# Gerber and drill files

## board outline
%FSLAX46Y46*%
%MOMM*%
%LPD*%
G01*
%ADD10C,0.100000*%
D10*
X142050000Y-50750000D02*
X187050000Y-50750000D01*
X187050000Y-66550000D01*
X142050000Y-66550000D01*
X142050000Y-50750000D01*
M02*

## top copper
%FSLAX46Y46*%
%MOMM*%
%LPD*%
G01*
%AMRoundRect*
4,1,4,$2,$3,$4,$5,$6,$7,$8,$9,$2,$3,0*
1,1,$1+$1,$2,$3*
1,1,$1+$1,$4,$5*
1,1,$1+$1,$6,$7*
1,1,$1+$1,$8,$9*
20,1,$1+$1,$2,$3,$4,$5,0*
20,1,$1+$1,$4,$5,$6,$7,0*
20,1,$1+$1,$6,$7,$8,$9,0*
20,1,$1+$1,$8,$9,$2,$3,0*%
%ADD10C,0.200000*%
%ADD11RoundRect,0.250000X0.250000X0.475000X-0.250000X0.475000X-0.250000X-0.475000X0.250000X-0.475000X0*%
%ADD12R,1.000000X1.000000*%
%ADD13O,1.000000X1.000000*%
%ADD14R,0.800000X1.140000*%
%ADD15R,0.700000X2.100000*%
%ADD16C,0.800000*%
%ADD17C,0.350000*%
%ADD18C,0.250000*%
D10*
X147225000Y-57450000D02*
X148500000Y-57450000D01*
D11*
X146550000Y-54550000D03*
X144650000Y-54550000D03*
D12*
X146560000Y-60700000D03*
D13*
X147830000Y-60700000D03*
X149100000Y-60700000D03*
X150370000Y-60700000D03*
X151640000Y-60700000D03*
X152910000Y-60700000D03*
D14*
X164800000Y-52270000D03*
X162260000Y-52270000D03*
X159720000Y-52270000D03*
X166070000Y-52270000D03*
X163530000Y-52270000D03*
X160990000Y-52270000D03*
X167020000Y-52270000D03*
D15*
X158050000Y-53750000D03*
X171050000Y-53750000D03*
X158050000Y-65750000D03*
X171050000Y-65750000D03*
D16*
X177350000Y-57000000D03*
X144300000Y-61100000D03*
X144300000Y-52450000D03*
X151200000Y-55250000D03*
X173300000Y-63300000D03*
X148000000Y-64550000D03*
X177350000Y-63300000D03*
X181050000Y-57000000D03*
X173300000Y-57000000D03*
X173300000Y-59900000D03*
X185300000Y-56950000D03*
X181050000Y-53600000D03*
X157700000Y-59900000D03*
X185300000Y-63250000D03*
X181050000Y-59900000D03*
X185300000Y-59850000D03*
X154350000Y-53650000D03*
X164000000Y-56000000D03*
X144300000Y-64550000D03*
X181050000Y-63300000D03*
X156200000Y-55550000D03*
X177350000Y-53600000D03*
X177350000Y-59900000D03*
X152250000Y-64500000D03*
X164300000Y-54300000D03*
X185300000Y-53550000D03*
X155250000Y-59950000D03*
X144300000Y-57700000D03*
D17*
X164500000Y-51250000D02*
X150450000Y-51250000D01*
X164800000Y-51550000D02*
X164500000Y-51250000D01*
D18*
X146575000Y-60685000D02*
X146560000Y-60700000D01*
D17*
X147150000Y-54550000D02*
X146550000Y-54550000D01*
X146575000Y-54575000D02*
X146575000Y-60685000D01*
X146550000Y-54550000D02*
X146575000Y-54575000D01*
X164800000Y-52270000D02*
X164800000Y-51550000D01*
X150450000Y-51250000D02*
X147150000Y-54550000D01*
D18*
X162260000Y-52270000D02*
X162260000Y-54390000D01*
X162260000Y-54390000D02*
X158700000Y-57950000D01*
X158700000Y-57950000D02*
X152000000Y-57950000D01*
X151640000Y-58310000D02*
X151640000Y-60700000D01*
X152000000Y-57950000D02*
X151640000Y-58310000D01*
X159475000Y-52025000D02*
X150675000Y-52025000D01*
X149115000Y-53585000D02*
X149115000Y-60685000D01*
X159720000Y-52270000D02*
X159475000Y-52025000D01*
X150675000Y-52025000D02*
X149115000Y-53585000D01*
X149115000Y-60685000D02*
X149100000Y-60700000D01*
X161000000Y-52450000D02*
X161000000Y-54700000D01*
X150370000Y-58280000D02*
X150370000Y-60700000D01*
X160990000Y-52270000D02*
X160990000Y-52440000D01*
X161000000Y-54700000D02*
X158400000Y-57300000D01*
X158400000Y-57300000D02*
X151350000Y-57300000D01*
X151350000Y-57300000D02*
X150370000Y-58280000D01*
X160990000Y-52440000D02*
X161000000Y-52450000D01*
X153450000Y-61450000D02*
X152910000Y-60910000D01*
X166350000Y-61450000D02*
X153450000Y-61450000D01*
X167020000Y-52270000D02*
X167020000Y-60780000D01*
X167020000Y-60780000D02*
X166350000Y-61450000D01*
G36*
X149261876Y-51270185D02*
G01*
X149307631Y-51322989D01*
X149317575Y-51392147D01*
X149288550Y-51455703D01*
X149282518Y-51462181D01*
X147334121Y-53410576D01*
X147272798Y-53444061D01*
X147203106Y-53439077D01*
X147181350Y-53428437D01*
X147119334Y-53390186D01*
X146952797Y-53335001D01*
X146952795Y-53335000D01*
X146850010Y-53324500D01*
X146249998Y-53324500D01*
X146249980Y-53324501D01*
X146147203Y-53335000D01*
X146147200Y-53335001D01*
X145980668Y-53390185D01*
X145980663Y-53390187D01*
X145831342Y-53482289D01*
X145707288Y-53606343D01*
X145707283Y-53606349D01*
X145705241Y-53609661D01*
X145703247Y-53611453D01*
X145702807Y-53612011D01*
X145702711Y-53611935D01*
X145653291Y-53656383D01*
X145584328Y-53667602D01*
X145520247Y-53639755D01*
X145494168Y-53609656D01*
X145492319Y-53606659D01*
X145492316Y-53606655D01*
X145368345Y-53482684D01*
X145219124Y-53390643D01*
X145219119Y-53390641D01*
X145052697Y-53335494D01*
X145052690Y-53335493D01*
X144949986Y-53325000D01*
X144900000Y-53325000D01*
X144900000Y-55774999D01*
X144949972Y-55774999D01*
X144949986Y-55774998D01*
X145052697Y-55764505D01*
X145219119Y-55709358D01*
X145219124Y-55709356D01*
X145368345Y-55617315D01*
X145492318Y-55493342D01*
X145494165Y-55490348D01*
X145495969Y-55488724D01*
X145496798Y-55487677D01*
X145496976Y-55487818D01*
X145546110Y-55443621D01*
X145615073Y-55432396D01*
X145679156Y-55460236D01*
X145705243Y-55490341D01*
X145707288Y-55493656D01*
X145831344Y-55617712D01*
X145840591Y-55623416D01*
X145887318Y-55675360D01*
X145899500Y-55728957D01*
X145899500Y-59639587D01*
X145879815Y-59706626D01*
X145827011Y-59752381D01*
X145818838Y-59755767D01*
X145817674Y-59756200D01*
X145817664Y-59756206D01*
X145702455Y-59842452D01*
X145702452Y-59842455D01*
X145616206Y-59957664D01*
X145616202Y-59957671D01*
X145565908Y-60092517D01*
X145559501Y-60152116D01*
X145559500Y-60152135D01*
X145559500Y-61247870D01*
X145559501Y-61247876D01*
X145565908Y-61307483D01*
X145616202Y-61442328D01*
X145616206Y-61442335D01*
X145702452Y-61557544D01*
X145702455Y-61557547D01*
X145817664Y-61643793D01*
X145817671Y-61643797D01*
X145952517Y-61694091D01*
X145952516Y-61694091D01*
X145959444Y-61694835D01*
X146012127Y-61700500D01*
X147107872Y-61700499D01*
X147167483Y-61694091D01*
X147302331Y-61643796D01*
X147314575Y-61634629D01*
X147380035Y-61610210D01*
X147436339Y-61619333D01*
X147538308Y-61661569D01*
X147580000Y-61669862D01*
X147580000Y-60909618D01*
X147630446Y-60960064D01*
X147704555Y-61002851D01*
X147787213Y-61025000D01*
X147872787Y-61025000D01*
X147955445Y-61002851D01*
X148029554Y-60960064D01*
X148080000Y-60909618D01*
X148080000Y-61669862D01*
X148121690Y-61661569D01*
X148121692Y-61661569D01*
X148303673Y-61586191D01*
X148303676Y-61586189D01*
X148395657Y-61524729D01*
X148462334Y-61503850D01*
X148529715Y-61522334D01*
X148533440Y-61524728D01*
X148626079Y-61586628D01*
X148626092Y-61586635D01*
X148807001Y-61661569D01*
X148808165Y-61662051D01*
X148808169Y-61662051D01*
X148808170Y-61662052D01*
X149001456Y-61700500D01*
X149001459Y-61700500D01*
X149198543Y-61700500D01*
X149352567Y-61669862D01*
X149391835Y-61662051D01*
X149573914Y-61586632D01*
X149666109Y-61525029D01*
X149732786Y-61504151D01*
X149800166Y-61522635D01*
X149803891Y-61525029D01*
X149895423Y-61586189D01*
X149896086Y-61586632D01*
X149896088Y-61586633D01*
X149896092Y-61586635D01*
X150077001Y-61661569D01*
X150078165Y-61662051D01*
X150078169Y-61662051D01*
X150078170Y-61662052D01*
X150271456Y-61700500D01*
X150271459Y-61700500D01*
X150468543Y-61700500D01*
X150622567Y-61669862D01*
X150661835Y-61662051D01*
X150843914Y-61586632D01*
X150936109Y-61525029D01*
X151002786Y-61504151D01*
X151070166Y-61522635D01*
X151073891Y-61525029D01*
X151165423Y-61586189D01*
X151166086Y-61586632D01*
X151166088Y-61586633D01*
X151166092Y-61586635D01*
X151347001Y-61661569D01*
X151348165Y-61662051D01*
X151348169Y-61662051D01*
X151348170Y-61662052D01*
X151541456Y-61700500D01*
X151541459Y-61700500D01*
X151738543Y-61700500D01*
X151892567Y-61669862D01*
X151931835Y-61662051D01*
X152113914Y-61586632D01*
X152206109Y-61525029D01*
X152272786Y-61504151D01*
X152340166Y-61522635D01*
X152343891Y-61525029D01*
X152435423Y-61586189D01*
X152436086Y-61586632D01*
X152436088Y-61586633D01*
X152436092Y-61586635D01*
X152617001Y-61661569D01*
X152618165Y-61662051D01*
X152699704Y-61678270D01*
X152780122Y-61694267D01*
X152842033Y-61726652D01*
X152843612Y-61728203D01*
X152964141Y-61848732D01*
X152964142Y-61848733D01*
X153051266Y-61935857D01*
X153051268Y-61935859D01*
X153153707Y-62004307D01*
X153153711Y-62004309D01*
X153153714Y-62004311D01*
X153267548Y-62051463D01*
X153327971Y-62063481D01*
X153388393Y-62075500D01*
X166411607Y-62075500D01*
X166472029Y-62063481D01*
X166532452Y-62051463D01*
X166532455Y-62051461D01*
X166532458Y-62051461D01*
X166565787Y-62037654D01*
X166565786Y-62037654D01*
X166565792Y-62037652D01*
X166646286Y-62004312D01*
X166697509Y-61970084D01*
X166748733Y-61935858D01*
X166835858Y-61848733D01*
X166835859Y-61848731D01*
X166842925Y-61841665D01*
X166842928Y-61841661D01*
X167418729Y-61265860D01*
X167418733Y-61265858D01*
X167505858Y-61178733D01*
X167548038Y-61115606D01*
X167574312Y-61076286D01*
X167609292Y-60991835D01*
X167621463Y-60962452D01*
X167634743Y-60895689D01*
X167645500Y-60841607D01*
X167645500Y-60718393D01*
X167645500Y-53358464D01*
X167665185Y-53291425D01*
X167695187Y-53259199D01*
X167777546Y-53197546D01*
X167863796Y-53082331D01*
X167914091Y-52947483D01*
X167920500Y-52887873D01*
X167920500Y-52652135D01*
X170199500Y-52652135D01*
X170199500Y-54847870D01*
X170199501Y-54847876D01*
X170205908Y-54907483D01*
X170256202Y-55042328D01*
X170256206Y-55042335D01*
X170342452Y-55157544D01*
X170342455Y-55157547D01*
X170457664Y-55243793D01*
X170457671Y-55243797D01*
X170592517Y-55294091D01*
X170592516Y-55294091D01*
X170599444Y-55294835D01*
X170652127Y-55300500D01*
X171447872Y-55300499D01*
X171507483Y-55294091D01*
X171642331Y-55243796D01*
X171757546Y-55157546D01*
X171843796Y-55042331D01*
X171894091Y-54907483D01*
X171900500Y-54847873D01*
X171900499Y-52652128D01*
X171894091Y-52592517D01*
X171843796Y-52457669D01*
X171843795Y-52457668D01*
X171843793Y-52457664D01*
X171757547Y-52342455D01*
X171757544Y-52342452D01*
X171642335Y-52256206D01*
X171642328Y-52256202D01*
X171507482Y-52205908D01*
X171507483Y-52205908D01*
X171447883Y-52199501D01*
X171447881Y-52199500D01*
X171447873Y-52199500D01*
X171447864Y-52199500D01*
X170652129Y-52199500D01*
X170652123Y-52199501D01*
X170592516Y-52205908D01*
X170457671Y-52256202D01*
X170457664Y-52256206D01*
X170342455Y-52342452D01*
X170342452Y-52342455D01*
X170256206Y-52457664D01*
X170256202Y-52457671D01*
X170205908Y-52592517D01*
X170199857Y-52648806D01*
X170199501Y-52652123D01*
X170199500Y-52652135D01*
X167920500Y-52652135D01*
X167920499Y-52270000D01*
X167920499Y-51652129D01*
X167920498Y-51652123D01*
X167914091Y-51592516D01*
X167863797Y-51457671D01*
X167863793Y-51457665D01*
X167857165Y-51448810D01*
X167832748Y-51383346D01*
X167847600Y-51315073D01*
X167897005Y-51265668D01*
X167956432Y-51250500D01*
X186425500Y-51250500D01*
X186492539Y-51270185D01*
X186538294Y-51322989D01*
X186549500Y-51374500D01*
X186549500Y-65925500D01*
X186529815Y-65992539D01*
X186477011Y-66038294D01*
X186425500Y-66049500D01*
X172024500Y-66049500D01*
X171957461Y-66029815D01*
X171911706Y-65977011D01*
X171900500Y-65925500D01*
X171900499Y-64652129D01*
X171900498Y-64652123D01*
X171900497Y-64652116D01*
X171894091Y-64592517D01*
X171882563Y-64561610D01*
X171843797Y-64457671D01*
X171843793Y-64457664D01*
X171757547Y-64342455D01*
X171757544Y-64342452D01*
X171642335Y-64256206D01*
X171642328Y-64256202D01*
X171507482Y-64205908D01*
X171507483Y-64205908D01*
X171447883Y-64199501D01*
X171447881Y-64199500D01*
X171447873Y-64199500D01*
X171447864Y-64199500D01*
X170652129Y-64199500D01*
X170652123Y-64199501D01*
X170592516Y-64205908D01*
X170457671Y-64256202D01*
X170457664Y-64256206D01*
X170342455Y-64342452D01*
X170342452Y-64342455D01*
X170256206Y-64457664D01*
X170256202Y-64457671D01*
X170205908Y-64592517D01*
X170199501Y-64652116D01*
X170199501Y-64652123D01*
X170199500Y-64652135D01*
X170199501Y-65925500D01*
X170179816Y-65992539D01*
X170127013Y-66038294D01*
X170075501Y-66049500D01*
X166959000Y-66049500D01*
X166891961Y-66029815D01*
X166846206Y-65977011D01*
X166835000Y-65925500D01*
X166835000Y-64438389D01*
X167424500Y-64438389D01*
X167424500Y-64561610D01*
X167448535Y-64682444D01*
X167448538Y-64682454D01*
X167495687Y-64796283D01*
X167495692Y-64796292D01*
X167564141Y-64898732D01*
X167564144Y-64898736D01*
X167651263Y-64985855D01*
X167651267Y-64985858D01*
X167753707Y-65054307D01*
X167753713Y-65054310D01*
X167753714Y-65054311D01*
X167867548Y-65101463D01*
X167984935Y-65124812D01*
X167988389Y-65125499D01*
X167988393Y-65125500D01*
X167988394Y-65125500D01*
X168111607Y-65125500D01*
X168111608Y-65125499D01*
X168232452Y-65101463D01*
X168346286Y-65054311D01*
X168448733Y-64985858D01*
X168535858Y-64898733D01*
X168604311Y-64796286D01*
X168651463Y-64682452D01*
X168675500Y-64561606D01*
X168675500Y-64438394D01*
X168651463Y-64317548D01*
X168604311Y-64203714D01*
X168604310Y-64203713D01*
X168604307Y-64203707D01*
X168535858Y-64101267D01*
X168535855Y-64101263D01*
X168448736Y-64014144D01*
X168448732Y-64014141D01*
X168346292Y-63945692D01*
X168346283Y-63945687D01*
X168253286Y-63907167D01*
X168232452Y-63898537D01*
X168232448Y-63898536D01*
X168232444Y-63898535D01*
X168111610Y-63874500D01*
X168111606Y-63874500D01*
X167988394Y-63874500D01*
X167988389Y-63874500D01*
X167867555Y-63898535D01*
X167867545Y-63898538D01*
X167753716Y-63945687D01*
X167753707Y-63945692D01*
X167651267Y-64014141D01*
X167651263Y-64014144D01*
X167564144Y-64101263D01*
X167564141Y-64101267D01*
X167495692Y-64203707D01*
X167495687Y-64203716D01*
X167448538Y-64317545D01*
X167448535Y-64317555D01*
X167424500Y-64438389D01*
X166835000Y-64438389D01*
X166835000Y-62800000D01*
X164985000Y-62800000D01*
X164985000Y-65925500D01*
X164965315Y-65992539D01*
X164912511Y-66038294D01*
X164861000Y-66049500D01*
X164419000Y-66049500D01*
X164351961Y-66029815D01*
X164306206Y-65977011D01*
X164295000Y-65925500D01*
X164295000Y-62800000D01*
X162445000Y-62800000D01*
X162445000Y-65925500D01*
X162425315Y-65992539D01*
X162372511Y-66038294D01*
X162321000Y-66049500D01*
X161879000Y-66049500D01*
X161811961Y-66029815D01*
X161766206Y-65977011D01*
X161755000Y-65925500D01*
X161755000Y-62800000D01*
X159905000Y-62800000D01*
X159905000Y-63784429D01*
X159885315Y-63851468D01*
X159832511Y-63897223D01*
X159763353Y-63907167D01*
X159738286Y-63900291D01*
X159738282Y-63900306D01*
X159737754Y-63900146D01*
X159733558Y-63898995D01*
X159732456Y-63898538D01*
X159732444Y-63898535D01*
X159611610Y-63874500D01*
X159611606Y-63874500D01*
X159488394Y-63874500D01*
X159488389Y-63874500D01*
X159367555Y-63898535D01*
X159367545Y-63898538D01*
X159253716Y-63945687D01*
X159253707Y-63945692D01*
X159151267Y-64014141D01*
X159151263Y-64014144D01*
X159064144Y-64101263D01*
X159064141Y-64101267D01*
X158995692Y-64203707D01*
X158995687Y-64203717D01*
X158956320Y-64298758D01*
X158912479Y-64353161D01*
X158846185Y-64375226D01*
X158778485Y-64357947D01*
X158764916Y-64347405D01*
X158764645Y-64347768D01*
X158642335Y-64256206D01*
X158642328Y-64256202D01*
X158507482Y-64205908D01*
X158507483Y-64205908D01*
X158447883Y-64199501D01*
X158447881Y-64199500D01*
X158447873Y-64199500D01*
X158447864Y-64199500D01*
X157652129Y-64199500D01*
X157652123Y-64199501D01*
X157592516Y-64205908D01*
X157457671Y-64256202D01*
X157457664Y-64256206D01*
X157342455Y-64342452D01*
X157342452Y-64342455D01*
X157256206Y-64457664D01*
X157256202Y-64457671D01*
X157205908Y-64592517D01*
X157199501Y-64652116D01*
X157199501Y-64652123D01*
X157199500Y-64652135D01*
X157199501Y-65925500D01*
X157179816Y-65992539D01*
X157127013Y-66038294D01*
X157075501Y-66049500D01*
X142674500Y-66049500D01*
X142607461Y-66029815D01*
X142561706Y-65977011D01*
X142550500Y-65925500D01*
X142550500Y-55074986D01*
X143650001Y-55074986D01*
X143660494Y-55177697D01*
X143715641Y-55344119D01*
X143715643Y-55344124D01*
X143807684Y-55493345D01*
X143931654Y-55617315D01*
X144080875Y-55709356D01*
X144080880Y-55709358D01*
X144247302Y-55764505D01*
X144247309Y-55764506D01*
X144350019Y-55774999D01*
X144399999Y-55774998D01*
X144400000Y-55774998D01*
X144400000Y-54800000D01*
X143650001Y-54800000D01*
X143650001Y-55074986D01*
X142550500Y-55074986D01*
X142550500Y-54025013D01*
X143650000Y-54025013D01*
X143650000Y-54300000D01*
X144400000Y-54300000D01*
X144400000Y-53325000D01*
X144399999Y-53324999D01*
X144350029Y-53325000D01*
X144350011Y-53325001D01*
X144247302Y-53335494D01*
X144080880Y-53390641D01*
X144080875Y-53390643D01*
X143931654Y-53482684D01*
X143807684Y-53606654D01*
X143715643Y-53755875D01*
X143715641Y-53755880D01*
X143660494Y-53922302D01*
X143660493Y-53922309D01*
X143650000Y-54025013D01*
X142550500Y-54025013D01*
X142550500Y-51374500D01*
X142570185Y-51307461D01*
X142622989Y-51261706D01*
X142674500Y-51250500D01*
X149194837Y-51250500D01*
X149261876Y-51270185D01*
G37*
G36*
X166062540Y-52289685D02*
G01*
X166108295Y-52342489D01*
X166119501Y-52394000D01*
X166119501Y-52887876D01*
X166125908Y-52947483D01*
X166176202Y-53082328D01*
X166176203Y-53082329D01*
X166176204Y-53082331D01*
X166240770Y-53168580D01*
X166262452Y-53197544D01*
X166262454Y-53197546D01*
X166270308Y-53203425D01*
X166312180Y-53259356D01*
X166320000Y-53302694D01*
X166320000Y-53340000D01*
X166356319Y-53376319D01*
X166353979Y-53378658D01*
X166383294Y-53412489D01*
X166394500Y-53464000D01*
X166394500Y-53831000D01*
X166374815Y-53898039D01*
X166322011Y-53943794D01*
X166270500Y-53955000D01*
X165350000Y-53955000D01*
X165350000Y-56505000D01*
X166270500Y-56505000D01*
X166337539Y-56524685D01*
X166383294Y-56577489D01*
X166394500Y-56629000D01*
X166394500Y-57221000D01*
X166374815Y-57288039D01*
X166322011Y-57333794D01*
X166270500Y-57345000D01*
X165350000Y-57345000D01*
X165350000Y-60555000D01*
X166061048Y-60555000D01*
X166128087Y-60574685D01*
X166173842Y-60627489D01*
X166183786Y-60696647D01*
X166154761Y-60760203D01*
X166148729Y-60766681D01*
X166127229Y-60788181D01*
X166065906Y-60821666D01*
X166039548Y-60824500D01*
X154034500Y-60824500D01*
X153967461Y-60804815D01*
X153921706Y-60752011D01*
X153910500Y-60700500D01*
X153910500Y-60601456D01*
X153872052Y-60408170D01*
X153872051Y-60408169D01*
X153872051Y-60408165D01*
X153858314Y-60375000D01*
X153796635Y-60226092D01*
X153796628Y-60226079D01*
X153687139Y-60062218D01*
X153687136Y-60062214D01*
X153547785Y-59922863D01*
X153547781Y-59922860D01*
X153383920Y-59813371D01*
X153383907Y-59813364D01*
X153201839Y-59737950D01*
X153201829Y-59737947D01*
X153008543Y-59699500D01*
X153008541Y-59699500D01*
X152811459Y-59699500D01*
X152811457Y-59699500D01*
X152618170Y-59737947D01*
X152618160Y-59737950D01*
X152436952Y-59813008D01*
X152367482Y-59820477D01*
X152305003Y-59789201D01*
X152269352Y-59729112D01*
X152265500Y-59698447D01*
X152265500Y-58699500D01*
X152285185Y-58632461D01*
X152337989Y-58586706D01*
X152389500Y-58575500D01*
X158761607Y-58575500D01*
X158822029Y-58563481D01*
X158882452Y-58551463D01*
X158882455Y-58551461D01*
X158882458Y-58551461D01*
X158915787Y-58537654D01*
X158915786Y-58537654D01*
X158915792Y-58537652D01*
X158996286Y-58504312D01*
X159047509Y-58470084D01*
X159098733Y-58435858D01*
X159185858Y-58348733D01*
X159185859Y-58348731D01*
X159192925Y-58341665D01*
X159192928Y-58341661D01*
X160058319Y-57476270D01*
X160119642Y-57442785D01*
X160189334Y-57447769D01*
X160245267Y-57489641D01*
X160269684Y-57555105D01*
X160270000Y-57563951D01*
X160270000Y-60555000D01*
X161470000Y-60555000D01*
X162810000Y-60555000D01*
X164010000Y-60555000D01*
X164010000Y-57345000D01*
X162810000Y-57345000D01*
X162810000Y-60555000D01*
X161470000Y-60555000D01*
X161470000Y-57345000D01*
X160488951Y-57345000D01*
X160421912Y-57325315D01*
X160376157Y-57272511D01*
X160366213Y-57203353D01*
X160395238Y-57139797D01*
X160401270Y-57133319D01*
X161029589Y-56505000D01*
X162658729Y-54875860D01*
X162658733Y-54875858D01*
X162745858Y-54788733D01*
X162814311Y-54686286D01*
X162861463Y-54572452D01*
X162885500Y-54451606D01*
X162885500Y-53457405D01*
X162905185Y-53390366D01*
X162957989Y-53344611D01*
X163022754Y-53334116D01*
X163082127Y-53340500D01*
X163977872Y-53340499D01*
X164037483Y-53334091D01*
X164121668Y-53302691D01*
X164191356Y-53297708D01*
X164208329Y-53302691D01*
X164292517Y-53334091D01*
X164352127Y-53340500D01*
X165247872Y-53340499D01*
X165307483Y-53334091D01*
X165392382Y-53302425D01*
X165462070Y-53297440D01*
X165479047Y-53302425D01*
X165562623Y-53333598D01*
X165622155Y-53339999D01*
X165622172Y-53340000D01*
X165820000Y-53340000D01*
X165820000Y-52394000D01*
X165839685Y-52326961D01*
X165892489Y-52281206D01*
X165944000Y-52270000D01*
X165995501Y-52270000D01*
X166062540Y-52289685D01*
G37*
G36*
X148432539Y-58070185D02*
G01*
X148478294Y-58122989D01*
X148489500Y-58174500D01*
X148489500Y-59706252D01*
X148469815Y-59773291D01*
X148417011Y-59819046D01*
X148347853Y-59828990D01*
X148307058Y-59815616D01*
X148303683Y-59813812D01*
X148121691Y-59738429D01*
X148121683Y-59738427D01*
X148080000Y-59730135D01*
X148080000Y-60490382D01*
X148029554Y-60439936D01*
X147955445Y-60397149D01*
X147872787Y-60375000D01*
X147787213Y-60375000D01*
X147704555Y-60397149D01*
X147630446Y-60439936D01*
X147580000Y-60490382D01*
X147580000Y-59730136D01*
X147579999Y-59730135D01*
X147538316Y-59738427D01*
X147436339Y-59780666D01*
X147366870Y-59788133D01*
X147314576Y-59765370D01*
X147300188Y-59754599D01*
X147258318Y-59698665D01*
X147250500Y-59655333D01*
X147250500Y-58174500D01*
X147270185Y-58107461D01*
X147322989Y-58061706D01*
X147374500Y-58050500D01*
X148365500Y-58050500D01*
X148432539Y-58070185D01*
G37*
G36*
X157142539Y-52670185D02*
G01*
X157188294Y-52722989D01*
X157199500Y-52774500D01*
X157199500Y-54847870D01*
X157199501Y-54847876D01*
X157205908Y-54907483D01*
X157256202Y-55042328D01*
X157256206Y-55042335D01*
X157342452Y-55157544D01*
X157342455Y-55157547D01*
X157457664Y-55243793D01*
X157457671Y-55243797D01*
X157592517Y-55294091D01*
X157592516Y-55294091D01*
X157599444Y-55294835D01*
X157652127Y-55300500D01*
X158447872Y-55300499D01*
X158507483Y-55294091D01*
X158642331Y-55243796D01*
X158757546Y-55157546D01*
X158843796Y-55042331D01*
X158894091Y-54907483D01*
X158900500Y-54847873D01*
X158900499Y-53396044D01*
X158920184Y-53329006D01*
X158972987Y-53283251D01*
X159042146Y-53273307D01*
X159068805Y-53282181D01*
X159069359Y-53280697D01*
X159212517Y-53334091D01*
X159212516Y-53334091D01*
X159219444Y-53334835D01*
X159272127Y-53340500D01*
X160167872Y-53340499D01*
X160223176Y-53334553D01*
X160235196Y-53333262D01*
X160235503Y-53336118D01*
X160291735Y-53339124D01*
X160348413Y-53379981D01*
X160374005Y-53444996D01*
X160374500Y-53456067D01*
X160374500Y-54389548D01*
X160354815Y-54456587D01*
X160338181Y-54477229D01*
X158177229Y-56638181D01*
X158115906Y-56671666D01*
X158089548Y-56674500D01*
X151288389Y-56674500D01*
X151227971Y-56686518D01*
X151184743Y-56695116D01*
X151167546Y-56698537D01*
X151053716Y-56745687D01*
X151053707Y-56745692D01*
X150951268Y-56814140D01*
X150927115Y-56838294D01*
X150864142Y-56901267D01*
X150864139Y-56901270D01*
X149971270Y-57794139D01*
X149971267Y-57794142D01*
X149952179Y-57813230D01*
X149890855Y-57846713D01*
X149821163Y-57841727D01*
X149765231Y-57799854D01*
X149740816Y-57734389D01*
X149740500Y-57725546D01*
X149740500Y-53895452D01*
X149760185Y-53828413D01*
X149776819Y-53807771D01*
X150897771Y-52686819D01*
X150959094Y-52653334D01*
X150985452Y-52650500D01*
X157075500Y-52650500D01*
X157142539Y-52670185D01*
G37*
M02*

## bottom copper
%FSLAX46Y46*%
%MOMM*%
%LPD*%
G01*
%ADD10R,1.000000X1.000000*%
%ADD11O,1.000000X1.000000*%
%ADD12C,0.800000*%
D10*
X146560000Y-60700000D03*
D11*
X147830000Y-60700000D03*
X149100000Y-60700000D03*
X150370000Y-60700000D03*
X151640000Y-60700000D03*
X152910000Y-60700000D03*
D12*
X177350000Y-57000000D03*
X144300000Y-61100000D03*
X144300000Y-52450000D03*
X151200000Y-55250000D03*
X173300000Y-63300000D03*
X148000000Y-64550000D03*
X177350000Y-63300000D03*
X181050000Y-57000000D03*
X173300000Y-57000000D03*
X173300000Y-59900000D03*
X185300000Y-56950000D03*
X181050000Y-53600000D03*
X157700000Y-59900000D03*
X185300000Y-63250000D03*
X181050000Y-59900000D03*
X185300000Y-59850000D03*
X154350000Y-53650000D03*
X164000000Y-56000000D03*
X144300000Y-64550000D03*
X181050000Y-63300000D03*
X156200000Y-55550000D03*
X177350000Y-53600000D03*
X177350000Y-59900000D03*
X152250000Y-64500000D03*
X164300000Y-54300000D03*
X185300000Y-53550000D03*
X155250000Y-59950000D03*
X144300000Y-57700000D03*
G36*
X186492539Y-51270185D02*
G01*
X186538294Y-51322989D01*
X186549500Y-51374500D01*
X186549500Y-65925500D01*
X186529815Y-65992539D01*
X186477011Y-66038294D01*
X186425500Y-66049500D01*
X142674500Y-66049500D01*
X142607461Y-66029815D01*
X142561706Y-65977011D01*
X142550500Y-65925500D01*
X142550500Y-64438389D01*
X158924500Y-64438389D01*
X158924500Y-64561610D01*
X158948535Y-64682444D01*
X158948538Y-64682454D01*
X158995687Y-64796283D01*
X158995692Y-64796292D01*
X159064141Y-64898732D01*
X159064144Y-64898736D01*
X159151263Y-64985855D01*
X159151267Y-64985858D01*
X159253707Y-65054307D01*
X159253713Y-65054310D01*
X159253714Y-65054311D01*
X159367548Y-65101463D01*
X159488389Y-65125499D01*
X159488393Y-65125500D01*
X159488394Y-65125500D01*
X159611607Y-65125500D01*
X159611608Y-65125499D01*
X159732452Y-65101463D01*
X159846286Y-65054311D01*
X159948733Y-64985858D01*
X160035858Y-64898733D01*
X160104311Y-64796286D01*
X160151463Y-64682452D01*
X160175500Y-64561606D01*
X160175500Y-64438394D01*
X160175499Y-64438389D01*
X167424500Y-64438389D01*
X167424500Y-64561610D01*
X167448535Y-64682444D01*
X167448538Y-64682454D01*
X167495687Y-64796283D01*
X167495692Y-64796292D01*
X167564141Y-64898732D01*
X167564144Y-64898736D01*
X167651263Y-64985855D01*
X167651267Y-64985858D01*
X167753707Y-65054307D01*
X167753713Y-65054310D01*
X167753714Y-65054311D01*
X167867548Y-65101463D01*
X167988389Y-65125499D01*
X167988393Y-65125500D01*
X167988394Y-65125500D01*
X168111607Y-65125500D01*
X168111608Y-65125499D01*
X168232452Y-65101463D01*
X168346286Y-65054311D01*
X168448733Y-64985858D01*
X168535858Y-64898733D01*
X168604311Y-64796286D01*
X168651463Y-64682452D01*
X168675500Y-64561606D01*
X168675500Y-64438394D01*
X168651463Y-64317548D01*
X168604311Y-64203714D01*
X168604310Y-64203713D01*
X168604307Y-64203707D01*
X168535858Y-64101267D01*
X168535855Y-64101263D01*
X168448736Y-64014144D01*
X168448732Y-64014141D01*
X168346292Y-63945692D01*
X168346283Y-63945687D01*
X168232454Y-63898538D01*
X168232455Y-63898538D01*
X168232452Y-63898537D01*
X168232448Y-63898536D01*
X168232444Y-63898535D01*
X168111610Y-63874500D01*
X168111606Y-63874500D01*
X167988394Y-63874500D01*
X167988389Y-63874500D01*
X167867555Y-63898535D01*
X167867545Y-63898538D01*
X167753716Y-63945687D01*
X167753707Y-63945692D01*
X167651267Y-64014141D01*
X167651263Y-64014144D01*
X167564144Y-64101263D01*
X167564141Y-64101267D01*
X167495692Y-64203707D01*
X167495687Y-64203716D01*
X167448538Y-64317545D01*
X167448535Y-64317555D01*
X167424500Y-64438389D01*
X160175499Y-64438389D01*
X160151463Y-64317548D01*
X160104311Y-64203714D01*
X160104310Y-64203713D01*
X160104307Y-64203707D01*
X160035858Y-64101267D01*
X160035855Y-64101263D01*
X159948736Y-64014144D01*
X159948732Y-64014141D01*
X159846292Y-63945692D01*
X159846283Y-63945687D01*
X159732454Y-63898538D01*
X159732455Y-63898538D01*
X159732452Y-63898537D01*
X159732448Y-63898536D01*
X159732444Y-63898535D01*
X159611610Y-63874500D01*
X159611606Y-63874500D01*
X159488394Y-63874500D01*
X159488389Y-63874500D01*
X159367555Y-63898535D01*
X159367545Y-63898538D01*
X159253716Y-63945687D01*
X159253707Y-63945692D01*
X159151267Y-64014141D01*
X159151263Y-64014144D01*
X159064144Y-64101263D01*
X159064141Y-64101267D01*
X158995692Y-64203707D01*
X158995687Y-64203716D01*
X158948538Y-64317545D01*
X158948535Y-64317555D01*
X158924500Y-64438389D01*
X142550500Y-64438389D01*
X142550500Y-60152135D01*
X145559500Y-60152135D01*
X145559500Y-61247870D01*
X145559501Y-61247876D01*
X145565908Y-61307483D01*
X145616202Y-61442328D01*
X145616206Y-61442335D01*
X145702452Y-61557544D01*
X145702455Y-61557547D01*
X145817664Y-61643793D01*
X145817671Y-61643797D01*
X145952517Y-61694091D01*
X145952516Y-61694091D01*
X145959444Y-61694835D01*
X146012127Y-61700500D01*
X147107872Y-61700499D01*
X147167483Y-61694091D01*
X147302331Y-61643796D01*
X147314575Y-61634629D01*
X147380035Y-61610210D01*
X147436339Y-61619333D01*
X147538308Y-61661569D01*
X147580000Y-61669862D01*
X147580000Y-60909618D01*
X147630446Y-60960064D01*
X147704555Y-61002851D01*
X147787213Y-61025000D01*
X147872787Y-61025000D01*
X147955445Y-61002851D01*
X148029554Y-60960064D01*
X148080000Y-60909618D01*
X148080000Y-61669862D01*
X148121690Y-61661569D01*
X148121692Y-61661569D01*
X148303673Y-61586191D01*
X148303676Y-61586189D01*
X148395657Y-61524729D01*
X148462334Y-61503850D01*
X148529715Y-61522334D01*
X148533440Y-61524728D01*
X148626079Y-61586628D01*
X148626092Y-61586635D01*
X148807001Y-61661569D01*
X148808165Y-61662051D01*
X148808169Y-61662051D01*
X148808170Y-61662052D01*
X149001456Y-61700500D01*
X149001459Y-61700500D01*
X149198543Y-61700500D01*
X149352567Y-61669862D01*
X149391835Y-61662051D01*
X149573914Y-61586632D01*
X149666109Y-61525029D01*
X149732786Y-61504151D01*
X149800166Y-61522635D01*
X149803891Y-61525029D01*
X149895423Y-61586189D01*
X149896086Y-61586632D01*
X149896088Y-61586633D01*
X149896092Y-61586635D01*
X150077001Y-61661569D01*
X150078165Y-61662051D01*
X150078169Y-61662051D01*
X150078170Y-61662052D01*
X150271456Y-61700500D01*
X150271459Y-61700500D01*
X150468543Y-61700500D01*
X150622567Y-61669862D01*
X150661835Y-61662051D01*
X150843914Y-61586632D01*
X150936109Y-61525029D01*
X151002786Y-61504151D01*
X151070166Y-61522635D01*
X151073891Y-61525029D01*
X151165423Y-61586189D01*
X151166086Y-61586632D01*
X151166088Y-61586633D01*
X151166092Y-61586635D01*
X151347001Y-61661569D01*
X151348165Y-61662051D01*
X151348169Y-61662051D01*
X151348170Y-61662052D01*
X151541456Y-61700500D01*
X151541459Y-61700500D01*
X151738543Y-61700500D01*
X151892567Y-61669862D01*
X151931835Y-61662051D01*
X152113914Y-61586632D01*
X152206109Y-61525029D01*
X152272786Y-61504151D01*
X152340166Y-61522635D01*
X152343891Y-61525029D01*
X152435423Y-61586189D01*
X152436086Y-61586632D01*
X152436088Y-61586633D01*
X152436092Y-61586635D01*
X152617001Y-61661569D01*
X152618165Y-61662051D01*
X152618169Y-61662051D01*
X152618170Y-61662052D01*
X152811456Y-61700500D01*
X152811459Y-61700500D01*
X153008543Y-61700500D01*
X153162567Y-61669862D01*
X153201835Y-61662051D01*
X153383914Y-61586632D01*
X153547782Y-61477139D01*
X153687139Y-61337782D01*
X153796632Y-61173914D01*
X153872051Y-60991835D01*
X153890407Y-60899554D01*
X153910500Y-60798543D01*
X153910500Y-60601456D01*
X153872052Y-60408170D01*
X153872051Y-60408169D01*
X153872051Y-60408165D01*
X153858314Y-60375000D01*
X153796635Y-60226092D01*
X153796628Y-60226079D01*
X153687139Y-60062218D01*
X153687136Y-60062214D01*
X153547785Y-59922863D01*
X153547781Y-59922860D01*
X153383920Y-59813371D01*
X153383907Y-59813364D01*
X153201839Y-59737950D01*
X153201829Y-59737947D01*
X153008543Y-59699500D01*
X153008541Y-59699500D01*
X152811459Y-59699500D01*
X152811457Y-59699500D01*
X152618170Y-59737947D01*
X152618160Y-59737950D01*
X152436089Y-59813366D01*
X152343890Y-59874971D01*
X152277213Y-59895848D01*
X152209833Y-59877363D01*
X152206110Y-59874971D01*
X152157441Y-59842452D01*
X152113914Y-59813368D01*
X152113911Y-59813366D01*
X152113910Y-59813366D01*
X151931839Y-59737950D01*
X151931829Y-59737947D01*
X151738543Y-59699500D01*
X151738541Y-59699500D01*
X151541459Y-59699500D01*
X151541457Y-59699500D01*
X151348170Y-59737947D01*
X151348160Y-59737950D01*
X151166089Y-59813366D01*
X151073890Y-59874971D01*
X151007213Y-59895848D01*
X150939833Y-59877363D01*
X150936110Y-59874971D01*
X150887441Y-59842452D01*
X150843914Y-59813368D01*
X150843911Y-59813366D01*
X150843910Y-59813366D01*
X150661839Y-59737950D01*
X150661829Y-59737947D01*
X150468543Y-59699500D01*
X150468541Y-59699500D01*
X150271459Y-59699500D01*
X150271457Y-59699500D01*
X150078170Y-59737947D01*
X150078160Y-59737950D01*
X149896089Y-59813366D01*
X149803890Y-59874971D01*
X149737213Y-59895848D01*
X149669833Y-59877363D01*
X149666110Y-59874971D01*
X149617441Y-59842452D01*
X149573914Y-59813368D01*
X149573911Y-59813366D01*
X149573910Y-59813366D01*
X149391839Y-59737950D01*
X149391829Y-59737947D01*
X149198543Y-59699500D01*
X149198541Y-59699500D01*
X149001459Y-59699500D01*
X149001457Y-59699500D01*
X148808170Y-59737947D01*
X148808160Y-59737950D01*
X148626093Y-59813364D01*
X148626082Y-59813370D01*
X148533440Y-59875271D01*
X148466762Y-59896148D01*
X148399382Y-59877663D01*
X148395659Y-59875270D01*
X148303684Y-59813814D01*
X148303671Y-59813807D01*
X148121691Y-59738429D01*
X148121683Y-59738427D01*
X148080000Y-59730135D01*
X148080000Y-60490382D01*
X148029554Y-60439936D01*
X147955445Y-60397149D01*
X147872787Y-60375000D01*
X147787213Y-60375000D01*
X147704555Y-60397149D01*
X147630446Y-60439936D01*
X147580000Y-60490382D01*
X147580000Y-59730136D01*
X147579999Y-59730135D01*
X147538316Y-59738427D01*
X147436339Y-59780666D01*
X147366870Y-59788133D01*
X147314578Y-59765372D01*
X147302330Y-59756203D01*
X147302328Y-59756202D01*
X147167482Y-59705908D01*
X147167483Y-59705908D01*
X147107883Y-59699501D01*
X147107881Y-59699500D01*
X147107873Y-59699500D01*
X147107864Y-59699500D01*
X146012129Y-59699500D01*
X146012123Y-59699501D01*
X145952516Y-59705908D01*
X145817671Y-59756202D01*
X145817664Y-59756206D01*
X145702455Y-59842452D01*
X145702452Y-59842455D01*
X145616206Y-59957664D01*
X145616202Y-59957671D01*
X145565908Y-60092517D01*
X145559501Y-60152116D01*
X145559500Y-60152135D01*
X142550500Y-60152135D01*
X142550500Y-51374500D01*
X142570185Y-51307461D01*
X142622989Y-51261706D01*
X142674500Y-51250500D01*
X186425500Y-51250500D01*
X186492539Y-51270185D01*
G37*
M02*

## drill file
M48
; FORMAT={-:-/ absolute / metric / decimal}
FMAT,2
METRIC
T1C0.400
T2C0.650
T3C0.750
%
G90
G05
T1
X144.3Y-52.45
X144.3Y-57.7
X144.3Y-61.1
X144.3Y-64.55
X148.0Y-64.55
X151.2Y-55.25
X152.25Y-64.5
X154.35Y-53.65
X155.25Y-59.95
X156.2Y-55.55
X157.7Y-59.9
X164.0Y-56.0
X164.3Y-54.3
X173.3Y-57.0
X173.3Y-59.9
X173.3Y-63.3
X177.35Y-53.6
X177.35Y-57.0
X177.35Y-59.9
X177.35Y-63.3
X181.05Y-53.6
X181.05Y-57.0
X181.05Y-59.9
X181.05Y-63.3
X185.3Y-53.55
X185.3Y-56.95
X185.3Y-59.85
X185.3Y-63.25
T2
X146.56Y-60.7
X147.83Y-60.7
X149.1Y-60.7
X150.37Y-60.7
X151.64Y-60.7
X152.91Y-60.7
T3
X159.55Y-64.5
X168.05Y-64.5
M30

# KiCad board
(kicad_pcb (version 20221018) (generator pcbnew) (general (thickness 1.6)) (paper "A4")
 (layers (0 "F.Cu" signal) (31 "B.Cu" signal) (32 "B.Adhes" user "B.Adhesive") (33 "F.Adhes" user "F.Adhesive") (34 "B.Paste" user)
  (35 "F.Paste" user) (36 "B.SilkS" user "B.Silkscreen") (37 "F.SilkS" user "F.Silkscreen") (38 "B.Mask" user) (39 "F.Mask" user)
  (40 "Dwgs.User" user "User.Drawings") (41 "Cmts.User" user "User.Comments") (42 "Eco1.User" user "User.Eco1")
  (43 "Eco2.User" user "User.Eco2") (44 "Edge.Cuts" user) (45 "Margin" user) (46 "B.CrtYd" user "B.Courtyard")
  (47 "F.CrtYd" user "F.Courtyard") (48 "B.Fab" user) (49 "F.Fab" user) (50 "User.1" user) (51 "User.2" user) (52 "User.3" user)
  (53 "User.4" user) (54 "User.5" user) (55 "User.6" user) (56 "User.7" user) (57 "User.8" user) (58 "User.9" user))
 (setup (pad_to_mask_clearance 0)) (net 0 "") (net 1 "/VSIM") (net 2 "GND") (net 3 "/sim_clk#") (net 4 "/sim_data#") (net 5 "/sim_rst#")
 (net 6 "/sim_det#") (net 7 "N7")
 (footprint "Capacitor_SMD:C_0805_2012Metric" (layer "F.Cu") (at 145.6 54.55 180)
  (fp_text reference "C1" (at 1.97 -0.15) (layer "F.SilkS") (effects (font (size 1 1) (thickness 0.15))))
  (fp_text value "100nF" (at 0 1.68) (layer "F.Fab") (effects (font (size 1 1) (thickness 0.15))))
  (pad "1" smd roundrect (at -0.95 0 180) (size 1 1.45) (layers "F.Cu" "F.Paste" "F.Mask") (roundrect_rratio 0.25) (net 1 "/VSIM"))
  (pad "2" smd roundrect (at 0.95 0 180) (size 1 1.45) (layers "F.Cu" "F.Paste" "F.Mask") (roundrect_rratio 0.25) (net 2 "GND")))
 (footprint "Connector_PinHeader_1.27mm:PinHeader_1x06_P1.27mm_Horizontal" (layer "F.Cu") (at 146.56 60.7 90)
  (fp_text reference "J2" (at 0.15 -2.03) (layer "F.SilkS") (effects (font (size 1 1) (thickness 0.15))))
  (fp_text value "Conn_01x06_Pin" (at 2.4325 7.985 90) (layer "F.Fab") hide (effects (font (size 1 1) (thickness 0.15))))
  (pad "1" thru_hole rect (at 0 0 90) (size 1 1) (drill 0.65) (layers "*.Cu" "*.Mask") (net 1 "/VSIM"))
  (pad "2" thru_hole oval (at 0 1.27 90) (size 1 1) (drill 0.65) (layers "*.Cu" "*.Mask") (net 2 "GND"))
  (pad "3" thru_hole oval (at 0 2.54 90) (size 1 1) (drill 0.65) (layers "*.Cu" "*.Mask") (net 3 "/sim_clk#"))
  (pad "4" thru_hole oval (at 0 3.81 90) (size 1 1) (drill 0.65) (layers "*.Cu" "*.Mask") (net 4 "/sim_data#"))
  (pad "5" thru_hole oval (at 0 5.08 90) (size 1 1) (drill 0.65) (layers "*.Cu" "*.Mask") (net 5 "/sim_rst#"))
  (pad "6" thru_hole oval (at 0 6.35 90) (size 1 1) (drill 0.65) (layers "*.Cu" "*.Mask") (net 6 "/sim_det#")))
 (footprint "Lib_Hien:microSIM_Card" (layer "F.Cu") (at 164.55 59.64)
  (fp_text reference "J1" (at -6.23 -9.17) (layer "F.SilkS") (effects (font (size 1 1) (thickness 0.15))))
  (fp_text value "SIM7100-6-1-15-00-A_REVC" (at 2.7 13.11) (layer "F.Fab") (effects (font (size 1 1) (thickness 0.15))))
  (pad "" np_thru_hole circle (at -5 4.86) (size 0.75 0.75) (drill 0.75) (layers "*.Cu" "*.Mask"))
  (pad "" np_thru_hole circle (at 3.5 4.86) (size 0.75 0.75) (drill 0.75) (layers "*.Cu" "*.Mask"))
  (pad "C1" smd rect (at 0.25 -7.37) (size 0.8 1.14) (layers "F.Cu" "F.Paste" "F.Mask") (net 1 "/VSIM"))
  (pad "C2" smd rect (at -2.29 -7.37) (size 0.8 1.14) (layers "F.Cu" "F.Paste" "F.Mask") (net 5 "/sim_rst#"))
  (pad "C3" smd rect (at -4.83 -7.37) (size 0.8 1.14) (layers "F.Cu" "F.Paste" "F.Mask") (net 3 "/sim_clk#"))
  (pad "C5" smd rect (at 1.52 -7.37) (size 0.8 1.14) (layers "F.Cu" "F.Paste" "F.Mask") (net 2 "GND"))
  (pad "C6" smd rect (at -1.02 -7.37) (size 0.8 1.14) (layers "F.Cu" "F.Paste" "F.Mask") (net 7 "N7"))
  (pad "C7" smd rect (at -3.56 -7.37) (size 0.8 1.14) (layers "F.Cu" "F.Paste" "F.Mask") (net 4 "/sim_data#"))
  (pad "CD" smd rect (at 2.47 -7.37) (size 0.8 1.14) (layers "F.Cu" "F.Paste" "F.Mask") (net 6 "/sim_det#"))
  (pad "G1" smd rect (at -6.5 -5.89) (size 0.7 2.1) (layers "F.Cu" "F.Paste" "F.Mask"))
  (pad "G2" smd rect (at 6.5 -5.89) (size 0.7 2.1) (layers "F.Cu" "F.Paste" "F.Mask"))
  (pad "G3" smd rect (at -6.5 6.11) (size 0.7 2.1) (layers "F.Cu" "F.Paste" "F.Mask"))
  (pad "G4" smd rect (at 6.5 6.11) (size 0.7 2.1) (layers "F.Cu" "F.Paste" "F.Mask"))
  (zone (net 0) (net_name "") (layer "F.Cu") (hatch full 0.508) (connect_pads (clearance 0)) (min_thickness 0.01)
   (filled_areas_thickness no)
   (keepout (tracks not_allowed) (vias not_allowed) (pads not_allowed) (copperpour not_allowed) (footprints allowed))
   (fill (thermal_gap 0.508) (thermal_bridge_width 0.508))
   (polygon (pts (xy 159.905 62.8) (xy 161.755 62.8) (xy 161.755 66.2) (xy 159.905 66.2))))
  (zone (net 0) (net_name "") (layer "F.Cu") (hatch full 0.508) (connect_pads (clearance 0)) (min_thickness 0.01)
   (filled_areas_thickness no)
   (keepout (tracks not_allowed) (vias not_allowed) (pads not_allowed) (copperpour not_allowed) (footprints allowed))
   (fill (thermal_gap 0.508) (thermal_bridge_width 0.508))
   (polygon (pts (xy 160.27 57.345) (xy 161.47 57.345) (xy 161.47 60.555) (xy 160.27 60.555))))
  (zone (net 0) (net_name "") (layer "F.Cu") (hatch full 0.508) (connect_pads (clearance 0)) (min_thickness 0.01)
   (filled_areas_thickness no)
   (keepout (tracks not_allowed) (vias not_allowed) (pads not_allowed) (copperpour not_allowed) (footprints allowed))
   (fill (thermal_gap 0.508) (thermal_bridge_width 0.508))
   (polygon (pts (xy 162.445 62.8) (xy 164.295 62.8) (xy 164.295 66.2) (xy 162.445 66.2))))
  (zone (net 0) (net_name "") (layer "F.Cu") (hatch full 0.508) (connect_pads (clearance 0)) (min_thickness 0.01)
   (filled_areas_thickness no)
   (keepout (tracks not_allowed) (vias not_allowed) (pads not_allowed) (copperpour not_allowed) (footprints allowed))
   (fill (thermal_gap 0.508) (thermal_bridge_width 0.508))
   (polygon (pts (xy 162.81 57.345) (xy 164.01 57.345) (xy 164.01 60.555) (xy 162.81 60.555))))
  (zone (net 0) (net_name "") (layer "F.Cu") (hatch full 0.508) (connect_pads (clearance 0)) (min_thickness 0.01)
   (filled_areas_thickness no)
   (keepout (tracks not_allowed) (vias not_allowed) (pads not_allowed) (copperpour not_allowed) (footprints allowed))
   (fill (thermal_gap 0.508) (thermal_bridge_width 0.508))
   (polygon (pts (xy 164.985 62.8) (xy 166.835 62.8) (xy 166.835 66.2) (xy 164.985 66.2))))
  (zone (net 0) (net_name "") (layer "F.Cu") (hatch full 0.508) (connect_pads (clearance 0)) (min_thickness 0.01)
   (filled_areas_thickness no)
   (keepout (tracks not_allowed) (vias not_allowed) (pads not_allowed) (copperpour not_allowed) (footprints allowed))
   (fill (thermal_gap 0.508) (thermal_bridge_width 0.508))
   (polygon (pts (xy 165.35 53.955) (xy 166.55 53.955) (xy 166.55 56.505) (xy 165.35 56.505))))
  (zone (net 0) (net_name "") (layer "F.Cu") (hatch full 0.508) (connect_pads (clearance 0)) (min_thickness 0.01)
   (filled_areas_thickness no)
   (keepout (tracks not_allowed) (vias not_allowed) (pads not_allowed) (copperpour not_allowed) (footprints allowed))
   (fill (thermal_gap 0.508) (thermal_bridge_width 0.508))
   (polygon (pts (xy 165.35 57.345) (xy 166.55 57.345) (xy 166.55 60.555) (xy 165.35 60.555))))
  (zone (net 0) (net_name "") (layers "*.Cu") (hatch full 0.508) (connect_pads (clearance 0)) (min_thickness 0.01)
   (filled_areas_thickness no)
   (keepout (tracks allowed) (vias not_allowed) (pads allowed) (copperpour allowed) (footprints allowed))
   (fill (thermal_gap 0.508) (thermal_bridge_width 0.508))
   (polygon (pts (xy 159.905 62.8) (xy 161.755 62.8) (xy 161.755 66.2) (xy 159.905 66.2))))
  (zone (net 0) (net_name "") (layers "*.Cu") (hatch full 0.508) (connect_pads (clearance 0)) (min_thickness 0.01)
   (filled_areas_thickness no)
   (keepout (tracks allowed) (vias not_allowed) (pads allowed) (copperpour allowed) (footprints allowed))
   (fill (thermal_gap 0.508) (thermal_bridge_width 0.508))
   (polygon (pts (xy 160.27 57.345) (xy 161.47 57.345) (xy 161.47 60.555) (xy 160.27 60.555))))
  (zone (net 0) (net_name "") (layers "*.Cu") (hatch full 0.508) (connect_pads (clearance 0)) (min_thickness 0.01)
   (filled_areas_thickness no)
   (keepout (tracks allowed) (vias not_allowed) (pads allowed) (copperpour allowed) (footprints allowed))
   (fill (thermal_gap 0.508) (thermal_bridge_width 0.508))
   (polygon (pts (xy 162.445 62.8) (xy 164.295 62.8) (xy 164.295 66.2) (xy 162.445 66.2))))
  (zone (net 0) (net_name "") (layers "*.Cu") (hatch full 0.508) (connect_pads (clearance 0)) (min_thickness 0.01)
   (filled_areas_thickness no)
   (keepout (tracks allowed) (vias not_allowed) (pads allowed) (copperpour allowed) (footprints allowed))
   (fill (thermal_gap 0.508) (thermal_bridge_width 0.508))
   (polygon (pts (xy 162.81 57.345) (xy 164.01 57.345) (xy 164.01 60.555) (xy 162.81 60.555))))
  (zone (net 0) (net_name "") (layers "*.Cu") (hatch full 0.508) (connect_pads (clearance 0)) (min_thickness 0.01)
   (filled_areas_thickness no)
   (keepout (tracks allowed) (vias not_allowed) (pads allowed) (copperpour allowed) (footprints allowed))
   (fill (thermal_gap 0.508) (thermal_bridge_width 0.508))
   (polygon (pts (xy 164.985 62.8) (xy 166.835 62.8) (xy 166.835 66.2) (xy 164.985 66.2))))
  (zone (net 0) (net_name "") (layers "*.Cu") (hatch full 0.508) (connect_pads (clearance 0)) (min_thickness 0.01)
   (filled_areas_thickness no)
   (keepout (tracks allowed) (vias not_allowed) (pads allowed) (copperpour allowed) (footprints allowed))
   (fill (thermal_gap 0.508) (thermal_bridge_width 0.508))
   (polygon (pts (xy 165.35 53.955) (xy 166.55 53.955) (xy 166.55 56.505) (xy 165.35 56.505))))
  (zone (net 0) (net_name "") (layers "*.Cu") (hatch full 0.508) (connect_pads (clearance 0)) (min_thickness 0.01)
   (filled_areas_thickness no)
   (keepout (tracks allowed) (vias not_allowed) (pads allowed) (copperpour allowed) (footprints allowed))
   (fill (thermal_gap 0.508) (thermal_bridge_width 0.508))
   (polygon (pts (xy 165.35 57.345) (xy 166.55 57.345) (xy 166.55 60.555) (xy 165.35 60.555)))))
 (gr_line (start 147.225 57.45) (end 148.5 57.45) (stroke (width 0.2) (type default)) (layer "F.Cu"))
 (gr_rect (start 142.05 50.75) (end 187.05 66.55) (stroke (width 0.1) (type default)) (fill none) (layer "Edge.Cuts"))
 (segment (start 164.5 51.25) (end 150.45 51.25) (width 0.35) (layer "F.Cu") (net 1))
 (segment (start 164.8 51.55) (end 164.5 51.25) (width 0.35) (layer "F.Cu") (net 1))
 (segment (start 146.575 60.685) (end 146.56 60.7) (width 0.25) (layer "F.Cu") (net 1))
 (segment (start 147.15 54.55) (end 146.55 54.55) (width 0.35) (layer "F.Cu") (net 1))
 (segment (start 146.575 54.575) (end 146.575 60.685) (width 0.35) (layer "F.Cu") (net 1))
 (segment (start 146.55 54.55) (end 146.575 54.575) (width 0.35) (layer "F.Cu") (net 1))
 (segment (start 164.8 52.27) (end 164.8 51.55) (width 0.35) (layer "F.Cu") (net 1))
 (segment (start 150.45 51.25) (end 147.15 54.55) (width 0.35) (layer "F.Cu") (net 1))
 (via (at 177.35 57) (size 0.8) (drill 0.4) (layers "F.Cu" "B.Cu") (free) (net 2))
 (via (at 144.3 61.1) (size 0.8) (drill 0.4) (layers "F.Cu" "B.Cu") (free) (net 2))
 (via (at 144.3 52.45) (size 0.8) (drill 0.4) (layers "F.Cu" "B.Cu") (free) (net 2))
 (via (at 151.2 55.25) (size 0.8) (drill 0.4) (layers "F.Cu" "B.Cu") (free) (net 2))
 (via (at 173.3 63.3) (size 0.8) (drill 0.4) (layers "F.Cu" "B.Cu") (free) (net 2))
 (via (at 148 64.55) (size 0.8) (drill 0.4) (layers "F.Cu" "B.Cu") (free) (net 2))
 (via (at 177.35 63.3) (size 0.8) (drill 0.4) (layers "F.Cu" "B.Cu") (free) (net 2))
 (via (at 181.05 57) (size 0.8) (drill 0.4) (layers "F.Cu" "B.Cu") (free) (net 2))
 (via (at 173.3 57) (size 0.8) (drill 0.4) (layers "F.Cu" "B.Cu") (free) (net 2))
 (via (at 173.3 59.9) (size 0.8) (drill 0.4) (layers "F.Cu" "B.Cu") (free) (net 2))
 (via (at 185.3 56.95) (size 0.8) (drill 0.4) (layers "F.Cu" "B.Cu") (free) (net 2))
 (via (at 181.05 53.6) (size 0.8) (drill 0.4) (layers "F.Cu" "B.Cu") (free) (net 2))
 (via (at 157.7 59.9) (size 0.8) (drill 0.4) (layers "F.Cu" "B.Cu") (free) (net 2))
 (via (at 185.3 63.25) (size 0.8) (drill 0.4) (layers "F.Cu" "B.Cu") (free) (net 2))
 (via (at 181.05 59.9) (size 0.8) (drill 0.4) (layers "F.Cu" "B.Cu") (free) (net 2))
 (via (at 185.3 59.85) (size 0.8) (drill 0.4) (layers "F.Cu" "B.Cu") (free) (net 2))
 (via (at 154.35 53.65) (size 0.8) (drill 0.4) (layers "F.Cu" "B.Cu") (free) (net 2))
 (via (at 164 56) (size 0.8) (drill 0.4) (layers "F.Cu" "B.Cu") (free) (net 2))
 (via (at 144.3 64.55) (size 0.8) (drill 0.4) (layers "F.Cu" "B.Cu") (free) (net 2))
 (via (at 181.05 63.3) (size 0.8) (drill 0.4) (layers "F.Cu" "B.Cu") (free) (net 2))
 (via (at 156.2 55.55) (size 0.8) (drill 0.4) (layers "F.Cu" "B.Cu") (free) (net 2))
 (via (at 177.35 53.6) (size 0.8) (drill 0.4) (layers "F.Cu" "B.Cu") (free) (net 2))
 (via (at 177.35 59.9) (size 0.8) (drill 0.4) (layers "F.Cu" "B.Cu") (free) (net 2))
 (via (at 152.25 64.5) (size 0.8) (drill 0.4) (layers "F.Cu" "B.Cu") (free) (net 2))
 (via (at 164.3 54.3) (size 0.8) (drill 0.4) (layers "F.Cu" "B.Cu") (free) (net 2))
 (via (at 185.3 53.55) (size 0.8) (drill 0.4) (layers "F.Cu" "B.Cu") (free) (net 2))
 (via (at 155.25 59.95) (size 0.8) (drill 0.4) (layers "F.Cu" "B.Cu") (free) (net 2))
 (via (at 144.3 57.7) (size 0.8) (drill 0.4) (layers "F.Cu" "B.Cu") (free) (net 2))
 (segment (start 162.26 52.27) (end 162.26 54.39) (width 0.25) (layer "F.Cu") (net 5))
 (segment (start 162.26 54.39) (end 158.7 57.95) (width 0.25) (layer "F.Cu") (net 5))
 (segment (start 158.7 57.95) (end 152 57.95) (width 0.25) (layer "F.Cu") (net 5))
 (segment (start 151.64 58.31) (end 151.64 60.7) (width 0.25) (layer "F.Cu") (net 5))
 (segment (start 152 57.95) (end 151.64 58.31) (width 0.25) (layer "F.Cu") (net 5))
 (segment (start 159.475 52.025) (end 150.675 52.025) (width 0.25) (layer "F.Cu") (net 3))
 (segment (start 149.115 53.585) (end 149.115 60.685) (width 0.25) (layer "F.Cu") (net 3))
 (segment (start 159.72 52.27) (end 159.475 52.025) (width 0.25) (layer "F.Cu") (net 3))
 (segment (start 150.675 52.025) (end 149.115 53.585) (width 0.25) (layer "F.Cu") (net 3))
 (segment (start 149.115 60.685) (end 149.1 60.7) (width 0.25) (layer "F.Cu") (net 3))
 (segment (start 161 52.45) (end 161 54.7) (width 0.25) (layer "F.Cu") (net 4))
 (segment (start 150.37 58.28) (end 150.37 60.7) (width 0.25) (layer "F.Cu") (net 4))
 (segment (start 160.99 52.27) (end 160.99 52.44) (width 0.25) (layer "F.Cu") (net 4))
 (segment (start 161 54.7) (end 158.4 57.3) (width 0.25) (layer "F.Cu") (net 4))
 (segment (start 158.4 57.3) (end 151.35 57.3) (width 0.25) (layer "F.Cu") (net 4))
 (segment (start 151.35 57.3) (end 150.37 58.28) (width 0.25) (layer "F.Cu") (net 4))
 (segment (start 160.99 52.44) (end 161 52.45) (width 0.25) (layer "F.Cu") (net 4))
 (segment (start 153.45 61.45) (end 152.91 60.91) (width 0.25) (layer "F.Cu") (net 6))
 (segment (start 166.35 61.45) (end 153.45 61.45) (width 0.25) (layer "F.Cu") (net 6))
 (segment (start 167.02 52.27) (end 167.02 60.78) (width 0.25) (layer "F.Cu") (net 6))
 (segment (start 167.02 60.78) (end 166.35 61.45) (width 0.25) (layer "F.Cu") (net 6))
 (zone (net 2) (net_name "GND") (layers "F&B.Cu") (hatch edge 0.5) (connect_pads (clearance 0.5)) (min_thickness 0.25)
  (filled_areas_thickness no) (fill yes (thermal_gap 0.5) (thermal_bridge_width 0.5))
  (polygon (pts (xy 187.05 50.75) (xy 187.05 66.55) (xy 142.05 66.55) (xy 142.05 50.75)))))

